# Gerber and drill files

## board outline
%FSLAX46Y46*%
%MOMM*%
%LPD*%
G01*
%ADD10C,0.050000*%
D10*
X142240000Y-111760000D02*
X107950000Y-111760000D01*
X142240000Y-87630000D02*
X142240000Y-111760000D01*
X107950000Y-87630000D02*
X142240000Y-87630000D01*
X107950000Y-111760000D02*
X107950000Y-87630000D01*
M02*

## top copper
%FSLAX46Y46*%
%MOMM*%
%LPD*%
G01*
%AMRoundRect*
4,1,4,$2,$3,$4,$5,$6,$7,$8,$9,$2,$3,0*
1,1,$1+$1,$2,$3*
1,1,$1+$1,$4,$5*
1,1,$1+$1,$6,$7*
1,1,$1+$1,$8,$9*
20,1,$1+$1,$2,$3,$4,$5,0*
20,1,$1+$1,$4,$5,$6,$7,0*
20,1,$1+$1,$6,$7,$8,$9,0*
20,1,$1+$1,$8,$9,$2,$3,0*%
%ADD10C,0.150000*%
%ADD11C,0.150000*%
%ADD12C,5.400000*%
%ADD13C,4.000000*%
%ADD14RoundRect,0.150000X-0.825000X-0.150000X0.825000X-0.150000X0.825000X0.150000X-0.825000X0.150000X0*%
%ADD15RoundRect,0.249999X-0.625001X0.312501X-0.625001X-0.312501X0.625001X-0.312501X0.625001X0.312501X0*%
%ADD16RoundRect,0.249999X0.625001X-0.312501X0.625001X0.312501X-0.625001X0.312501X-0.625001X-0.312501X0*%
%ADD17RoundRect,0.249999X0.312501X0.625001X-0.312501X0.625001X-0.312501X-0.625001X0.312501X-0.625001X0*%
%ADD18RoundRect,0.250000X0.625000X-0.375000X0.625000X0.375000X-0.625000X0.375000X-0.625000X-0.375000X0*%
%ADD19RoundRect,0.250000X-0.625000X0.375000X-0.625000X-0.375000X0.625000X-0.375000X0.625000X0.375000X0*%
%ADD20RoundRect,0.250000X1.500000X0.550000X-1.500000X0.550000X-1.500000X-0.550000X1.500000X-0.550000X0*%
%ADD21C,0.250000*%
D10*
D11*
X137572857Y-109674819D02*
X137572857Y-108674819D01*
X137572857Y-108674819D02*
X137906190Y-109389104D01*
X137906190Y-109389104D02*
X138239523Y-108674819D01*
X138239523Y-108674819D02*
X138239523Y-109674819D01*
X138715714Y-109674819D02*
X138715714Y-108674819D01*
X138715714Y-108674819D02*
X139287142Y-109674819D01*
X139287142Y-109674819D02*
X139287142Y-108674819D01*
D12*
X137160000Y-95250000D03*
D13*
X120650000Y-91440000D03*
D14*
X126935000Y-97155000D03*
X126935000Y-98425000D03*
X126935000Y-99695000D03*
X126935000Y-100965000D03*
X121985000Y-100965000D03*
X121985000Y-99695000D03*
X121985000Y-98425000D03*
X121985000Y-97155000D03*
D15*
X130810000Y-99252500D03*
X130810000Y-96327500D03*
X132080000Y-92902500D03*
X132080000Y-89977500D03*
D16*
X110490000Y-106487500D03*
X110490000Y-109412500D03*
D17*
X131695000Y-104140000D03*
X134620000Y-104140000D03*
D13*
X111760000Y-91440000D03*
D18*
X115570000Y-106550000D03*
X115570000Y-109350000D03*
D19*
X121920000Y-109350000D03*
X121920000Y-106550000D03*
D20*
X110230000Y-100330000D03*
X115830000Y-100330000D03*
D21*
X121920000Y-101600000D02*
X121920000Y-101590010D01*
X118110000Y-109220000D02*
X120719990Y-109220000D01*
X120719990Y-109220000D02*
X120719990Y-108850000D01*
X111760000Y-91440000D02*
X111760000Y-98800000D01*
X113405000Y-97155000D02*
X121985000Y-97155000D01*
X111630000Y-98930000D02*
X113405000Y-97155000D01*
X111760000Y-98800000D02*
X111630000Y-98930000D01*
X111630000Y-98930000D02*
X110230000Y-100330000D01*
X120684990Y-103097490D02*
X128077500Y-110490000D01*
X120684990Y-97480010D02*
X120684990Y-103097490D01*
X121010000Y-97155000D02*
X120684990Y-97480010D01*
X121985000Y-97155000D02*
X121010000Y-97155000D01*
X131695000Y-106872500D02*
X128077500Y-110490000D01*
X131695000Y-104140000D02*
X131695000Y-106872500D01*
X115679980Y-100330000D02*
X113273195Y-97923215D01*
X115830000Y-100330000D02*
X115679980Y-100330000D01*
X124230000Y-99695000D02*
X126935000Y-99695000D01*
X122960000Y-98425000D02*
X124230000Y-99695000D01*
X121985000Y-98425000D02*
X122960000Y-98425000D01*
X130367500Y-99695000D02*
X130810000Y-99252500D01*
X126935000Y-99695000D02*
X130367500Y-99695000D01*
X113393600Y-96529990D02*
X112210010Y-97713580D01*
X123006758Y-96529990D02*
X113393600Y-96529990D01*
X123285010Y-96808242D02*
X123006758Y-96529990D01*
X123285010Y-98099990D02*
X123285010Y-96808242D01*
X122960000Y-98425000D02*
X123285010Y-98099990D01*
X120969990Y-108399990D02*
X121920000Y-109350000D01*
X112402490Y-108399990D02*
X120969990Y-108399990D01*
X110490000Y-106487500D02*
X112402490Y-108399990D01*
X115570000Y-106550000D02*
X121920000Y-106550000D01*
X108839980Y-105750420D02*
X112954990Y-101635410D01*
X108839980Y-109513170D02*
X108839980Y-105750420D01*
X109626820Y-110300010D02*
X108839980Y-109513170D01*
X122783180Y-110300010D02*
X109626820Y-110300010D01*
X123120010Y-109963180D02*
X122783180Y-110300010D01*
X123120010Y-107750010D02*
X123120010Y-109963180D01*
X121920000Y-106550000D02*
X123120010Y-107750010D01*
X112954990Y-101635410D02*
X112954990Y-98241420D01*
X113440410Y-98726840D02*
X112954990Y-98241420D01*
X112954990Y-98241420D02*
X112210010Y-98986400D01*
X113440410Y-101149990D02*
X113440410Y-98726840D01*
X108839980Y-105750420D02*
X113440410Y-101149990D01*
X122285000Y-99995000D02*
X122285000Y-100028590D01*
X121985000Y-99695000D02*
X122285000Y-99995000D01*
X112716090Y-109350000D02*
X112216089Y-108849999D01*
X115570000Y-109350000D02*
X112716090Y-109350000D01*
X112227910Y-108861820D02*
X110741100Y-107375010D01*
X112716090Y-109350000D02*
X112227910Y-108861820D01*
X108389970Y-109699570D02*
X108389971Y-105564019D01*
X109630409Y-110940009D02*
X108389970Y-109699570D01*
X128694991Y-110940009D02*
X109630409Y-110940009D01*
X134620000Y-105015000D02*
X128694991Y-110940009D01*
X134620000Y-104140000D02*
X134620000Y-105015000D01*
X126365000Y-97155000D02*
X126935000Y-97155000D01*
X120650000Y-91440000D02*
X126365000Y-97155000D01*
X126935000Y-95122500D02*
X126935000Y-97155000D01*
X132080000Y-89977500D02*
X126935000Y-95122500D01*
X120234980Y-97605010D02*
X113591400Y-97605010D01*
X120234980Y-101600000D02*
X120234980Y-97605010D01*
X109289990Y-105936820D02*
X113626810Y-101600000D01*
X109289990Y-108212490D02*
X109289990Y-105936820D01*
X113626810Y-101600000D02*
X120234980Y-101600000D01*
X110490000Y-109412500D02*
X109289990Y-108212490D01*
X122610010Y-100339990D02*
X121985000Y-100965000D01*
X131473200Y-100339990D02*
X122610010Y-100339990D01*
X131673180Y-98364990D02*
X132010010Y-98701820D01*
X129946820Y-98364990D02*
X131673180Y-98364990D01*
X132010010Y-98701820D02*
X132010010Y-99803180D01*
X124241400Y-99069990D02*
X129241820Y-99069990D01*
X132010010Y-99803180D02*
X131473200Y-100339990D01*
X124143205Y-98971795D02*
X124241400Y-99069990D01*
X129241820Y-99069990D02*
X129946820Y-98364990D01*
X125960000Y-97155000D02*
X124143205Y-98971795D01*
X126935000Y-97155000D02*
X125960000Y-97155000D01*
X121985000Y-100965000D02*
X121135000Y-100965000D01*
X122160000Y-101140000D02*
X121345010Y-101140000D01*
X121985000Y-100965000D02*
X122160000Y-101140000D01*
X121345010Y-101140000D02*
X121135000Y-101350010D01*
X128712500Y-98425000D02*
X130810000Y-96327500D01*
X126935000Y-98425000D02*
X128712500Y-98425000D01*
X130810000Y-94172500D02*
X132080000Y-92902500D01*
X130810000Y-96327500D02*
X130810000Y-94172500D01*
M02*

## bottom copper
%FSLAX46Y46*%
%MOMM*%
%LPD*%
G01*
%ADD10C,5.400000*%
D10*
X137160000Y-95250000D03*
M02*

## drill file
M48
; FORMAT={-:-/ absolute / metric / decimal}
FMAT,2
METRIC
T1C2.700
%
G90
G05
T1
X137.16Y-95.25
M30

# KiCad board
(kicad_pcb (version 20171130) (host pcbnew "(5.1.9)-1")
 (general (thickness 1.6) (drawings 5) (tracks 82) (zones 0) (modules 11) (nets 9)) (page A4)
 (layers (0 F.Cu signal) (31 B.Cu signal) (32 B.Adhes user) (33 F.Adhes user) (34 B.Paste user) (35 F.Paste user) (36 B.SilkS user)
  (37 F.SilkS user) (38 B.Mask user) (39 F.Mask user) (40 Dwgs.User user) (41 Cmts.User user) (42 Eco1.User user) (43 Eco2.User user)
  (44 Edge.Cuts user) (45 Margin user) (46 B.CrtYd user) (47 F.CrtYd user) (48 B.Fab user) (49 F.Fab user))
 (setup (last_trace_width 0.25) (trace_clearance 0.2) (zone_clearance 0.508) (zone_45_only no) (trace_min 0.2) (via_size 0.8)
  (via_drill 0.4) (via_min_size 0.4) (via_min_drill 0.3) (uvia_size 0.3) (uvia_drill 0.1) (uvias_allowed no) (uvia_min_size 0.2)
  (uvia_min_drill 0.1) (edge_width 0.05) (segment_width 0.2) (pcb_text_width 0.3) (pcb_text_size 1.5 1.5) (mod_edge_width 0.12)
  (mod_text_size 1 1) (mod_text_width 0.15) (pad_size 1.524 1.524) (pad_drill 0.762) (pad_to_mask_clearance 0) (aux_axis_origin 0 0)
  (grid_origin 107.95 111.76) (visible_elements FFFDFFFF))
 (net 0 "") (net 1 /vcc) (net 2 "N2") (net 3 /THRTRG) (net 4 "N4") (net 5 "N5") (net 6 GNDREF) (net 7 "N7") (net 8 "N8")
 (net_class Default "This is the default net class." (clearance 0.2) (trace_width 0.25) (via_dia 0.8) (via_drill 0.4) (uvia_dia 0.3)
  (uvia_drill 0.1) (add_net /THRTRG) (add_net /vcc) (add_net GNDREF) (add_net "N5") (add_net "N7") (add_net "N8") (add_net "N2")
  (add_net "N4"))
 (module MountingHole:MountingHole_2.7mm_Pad (layer F.Cu) (at 137.16 95.25)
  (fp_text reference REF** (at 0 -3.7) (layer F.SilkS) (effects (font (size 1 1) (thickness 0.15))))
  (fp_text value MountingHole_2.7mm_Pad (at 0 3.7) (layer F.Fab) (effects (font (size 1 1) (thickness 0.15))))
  (pad 1 thru_hole circle (at 0 0) (size 5.4 5.4) (drill 2.7) (layers *.Cu *.Mask)))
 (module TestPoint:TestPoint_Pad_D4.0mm (layer F.Cu) (at 120.65 91.44)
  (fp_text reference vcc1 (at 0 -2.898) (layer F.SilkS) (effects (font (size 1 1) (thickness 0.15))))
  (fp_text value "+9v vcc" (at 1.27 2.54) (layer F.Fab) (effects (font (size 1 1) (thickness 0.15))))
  (pad 1 smd circle (at 0 0) (size 4 4) (layers F.Cu F.Mask) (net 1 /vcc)))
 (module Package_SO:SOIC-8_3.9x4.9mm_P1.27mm (layer F.Cu) (at 124.46 99.06)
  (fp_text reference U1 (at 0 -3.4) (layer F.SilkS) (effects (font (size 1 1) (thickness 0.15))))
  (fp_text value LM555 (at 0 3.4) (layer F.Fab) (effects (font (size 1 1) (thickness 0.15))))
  (pad 8 smd roundrect (at 2.475 -1.905) (size 1.95 0.6) (layers F.Cu F.Paste F.Mask) (roundrect_rratio 0.25) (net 1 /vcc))
  (pad 7 smd roundrect (at 2.475 -0.635) (size 1.95 0.6) (layers F.Cu F.Paste F.Mask) (roundrect_rratio 0.25) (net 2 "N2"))
  (pad 6 smd roundrect (at 2.475 0.635) (size 1.95 0.6) (layers F.Cu F.Paste F.Mask) (roundrect_rratio 0.25) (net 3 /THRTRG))
  (pad 5 smd roundrect (at 2.475 1.905) (size 1.95 0.6) (layers F.Cu F.Paste F.Mask) (roundrect_rratio 0.25) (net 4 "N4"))
  (pad 4 smd roundrect (at -2.475 1.905) (size 1.95 0.6) (layers F.Cu F.Paste F.Mask) (roundrect_rratio 0.25) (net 1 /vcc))
  (pad 3 smd roundrect (at -2.475 0.635) (size 1.95 0.6) (layers F.Cu F.Paste F.Mask) (roundrect_rratio 0.25) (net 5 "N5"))
  (pad 2 smd roundrect (at -2.475 -0.635) (size 1.95 0.6) (layers F.Cu F.Paste F.Mask) (roundrect_rratio 0.25) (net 3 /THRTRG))
  (pad 1 smd roundrect (at -2.475 -1.905) (size 1.95 0.6) (layers F.Cu F.Paste F.Mask) (roundrect_rratio 0.25) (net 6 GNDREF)))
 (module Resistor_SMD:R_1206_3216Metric (layer F.Cu) (at 130.81 97.79 270)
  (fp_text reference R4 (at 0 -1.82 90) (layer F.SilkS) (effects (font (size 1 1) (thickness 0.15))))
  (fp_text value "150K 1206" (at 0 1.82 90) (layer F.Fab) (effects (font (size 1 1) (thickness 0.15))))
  (pad 2 smd roundrect (at 1.4625 0 270) (size 1.125 1.75) (layers F.Cu F.Paste F.Mask) (roundrect_rratio 0.2222213333333333)
   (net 3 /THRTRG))
  (pad 1 smd roundrect (at -1.4625 0 270) (size 1.125 1.75) (layers F.Cu F.Paste F.Mask) (roundrect_rratio 0.2222213333333333) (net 2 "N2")))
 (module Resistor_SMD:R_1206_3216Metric (layer F.Cu) (at 132.08 91.44 270)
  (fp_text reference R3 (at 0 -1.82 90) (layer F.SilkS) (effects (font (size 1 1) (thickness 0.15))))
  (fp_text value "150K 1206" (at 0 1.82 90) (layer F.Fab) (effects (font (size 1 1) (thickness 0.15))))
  (pad 2 smd roundrect (at 1.4625 0 270) (size 1.125 1.75) (layers F.Cu F.Paste F.Mask) (roundrect_rratio 0.2222213333333333) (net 2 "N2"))
  (pad 1 smd roundrect (at -1.4625 0 270) (size 1.125 1.75) (layers F.Cu F.Paste F.Mask) (roundrect_rratio 0.2222213333333333) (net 1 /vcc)))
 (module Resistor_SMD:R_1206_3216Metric (layer F.Cu) (at 110.49 107.95 90)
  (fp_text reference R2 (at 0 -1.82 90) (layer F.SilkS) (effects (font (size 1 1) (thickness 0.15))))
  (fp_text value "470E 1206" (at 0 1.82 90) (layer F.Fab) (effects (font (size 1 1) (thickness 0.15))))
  (pad 2 smd roundrect (at 1.4625 0 90) (size 1.125 1.75) (layers F.Cu F.Paste F.Mask) (roundrect_rratio 0.2222213333333333) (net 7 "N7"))
  (pad 1 smd roundrect (at -1.4625 0 90) (size 1.125 1.75) (layers F.Cu F.Paste F.Mask) (roundrect_rratio 0.2222213333333333) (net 1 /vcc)))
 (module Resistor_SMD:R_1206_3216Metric (layer F.Cu) (at 133.1575 104.14 180)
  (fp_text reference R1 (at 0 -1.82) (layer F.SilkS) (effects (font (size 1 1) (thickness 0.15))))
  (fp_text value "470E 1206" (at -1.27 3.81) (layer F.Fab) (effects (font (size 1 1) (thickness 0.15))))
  (pad 2 smd roundrect (at 1.4625 0 180) (size 1.125 1.75) (layers F.Cu F.Paste F.Mask) (roundrect_rratio 0.2222213333333333) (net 6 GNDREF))
  (pad 1 smd roundrect (at -1.4625 0 180) (size 1.125 1.75) (layers F.Cu F.Paste F.Mask) (roundrect_rratio 0.2222213333333333) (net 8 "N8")))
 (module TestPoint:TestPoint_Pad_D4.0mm (layer F.Cu) (at 111.76 91.44)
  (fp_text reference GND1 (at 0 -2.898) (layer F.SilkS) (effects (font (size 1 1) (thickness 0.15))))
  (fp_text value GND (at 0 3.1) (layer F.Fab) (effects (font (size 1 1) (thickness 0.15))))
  (pad 1 smd circle (at 0 0) (size 4 4) (layers F.Cu F.Mask) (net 6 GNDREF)))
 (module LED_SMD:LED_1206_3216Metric (layer F.Cu) (at 115.57 107.95 90)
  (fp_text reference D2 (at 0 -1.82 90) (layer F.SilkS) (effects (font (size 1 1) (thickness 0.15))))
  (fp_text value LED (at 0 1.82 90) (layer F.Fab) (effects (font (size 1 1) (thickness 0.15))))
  (pad 2 smd roundrect (at 1.4 0 90) (size 1.25 1.75) (layers F.Cu F.Paste F.Mask) (roundrect_rratio 0.2) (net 5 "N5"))
  (pad 1 smd roundrect (at -1.4 0 90) (size 1.25 1.75) (layers F.Cu F.Paste F.Mask) (roundrect_rratio 0.2) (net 8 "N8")))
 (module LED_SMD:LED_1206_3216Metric (layer F.Cu) (at 121.92 107.95 270)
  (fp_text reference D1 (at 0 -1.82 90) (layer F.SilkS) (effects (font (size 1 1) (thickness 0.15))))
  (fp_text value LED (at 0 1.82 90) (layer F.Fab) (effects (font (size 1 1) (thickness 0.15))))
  (pad 2 smd roundrect (at 1.4 0 270) (size 1.25 1.75) (layers F.Cu F.Paste F.Mask) (roundrect_rratio 0.2) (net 7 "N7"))
  (pad 1 smd roundrect (at -1.4 0 270) (size 1.25 1.75) (layers F.Cu F.Paste F.Mask) (roundrect_rratio 0.2) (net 5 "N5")))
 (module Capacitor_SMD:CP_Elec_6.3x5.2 (layer F.Cu) (at 113.03 100.33 180)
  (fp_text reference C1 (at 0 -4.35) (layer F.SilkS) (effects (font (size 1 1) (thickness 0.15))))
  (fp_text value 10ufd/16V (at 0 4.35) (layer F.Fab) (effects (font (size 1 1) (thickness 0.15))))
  (pad 2 smd roundrect (at 2.8 0 180) (size 3.5 1.6) (layers F.Cu F.Paste F.Mask) (roundrect_rratio 0.15625) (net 6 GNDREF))
  (pad 1 smd roundrect (at -2.8 0 180) (size 3.5 1.6) (layers F.Cu F.Paste F.Mask) (roundrect_rratio 0.15625) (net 3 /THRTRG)))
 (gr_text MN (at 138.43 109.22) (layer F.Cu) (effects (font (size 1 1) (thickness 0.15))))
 (gr_line (start 142.24 111.76) (end 107.95 111.76) (layer Edge.Cuts) (width 0.05))
 (gr_line (start 142.24 87.63) (end 142.24 111.76) (layer Edge.Cuts) (width 0.05))
 (gr_line (start 107.95 87.63) (end 142.24 87.63) (layer Edge.Cuts) (width 0.05))
 (gr_line (start 107.95 111.76) (end 107.95 87.63) (layer Edge.Cuts) (width 0.05))
 (segment (start 121.92 101.6) (end 121.92 101.59001) (width 0.25) (layer F.Cu) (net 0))
 (segment (start 118.11 109.22) (end 120.71999 109.22) (width 0.25) (layer F.Cu) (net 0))
 (segment (start 120.71999 109.22) (end 120.71999 108.85) (width 0.25) (layer F.Cu) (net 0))
 (segment (start 111.76 91.44) (end 111.76 98.8) (width 0.25) (layer F.Cu) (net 6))
 (segment (start 113.405 97.155) (end 121.985 97.155) (width 0.25) (layer F.Cu) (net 6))
 (segment (start 111.63 98.93) (end 113.405 97.155) (width 0.25) (layer F.Cu) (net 6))
 (segment (start 111.76 98.8) (end 111.63 98.93) (width 0.25) (layer F.Cu) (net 6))
 (segment (start 111.63 98.93) (end 110.23 100.33) (width 0.25) (layer F.Cu) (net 6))
 (segment (start 120.68499 103.09749) (end 128.0775 110.49) (width 0.25) (layer F.Cu) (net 6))
 (segment (start 120.68499 97.48001) (end 120.68499 103.09749) (width 0.25) (layer F.Cu) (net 6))
 (segment (start 121.01 97.155) (end 120.68499 97.48001) (width 0.25) (layer F.Cu) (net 6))
 (segment (start 121.985 97.155) (end 121.01 97.155) (width 0.25) (layer F.Cu) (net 6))
 (segment (start 131.695 106.8725) (end 128.0775 110.49) (width 0.25) (layer F.Cu) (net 6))
 (segment (start 131.695 104.14) (end 131.695 106.8725) (width 0.25) (layer F.Cu) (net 6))
 (segment (start 115.67998 100.33) (end 113.273195 97.923215) (width 0.25) (layer F.Cu) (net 3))
 (segment (start 115.83 100.33) (end 115.67998 100.33) (width 0.25) (layer F.Cu) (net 3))
 (segment (start 124.23 99.695) (end 126.935 99.695) (width 0.25) (layer F.Cu) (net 3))
 (segment (start 122.96 98.425) (end 124.23 99.695) (width 0.25) (layer F.Cu) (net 3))
 (segment (start 121.985 98.425) (end 122.96 98.425) (width 0.25) (layer F.Cu) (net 3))
 (segment (start 130.3675 99.695) (end 130.81 99.2525) (width 0.25) (layer F.Cu) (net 3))
 (segment (start 126.935 99.695) (end 130.3675 99.695) (width 0.25) (layer F.Cu) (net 3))
 (segment (start 113.3936 96.52999) (end 112.21001 97.71358) (width 0.25) (layer F.Cu) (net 3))
 (segment (start 123.006758 96.52999) (end 113.3936 96.52999) (width 0.25) (layer F.Cu) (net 3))
 (segment (start 123.28501 96.808242) (end 123.006758 96.52999) (width 0.25) (layer F.Cu) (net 3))
 (segment (start 123.28501 98.09999) (end 123.28501 96.808242) (width 0.25) (layer F.Cu) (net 3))
 (segment (start 122.96 98.425) (end 123.28501 98.09999) (width 0.25) (layer F.Cu) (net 3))
 (segment (start 120.96999 108.39999) (end 121.92 109.35) (width 0.25) (layer F.Cu) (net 7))
 (segment (start 112.40249 108.39999) (end 120.96999 108.39999) (width 0.25) (layer F.Cu) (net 7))
 (segment (start 110.49 106.4875) (end 112.40249 108.39999) (width 0.25) (layer F.Cu) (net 7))
 (segment (start 115.57 106.55) (end 121.92 106.55) (width 0.25) (layer F.Cu) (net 5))
 (segment (start 108.83998 105.75042) (end 112.95499 101.63541) (width 0.25) (layer F.Cu) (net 5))
 (segment (start 108.83998 109.51317) (end 108.83998 105.75042) (width 0.25) (layer F.Cu) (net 5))
 (segment (start 109.62682 110.30001) (end 108.83998 109.51317) (width 0.25) (layer F.Cu) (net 5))
 (segment (start 122.78318 110.30001) (end 109.62682 110.30001) (width 0.25) (layer F.Cu) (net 5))
 (segment (start 123.12001 109.96318) (end 122.78318 110.30001) (width 0.25) (layer F.Cu) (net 5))
 (segment (start 123.12001 107.75001) (end 123.12001 109.96318) (width 0.25) (layer F.Cu) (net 5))
 (segment (start 121.92 106.55) (end 123.12001 107.75001) (width 0.25) (layer F.Cu) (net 5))
 (segment (start 112.95499 101.63541) (end 112.95499 98.24142) (width 0.25) (layer F.Cu) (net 5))
 (segment (start 113.44041 98.72684) (end 112.95499 98.24142) (width 0.25) (layer F.Cu) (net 5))
 (segment (start 112.95499 98.24142) (end 112.21001 98.9864) (width 0.25) (layer F.Cu) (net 5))
 (segment (start 113.44041 101.14999) (end 113.44041 98.72684) (width 0.25) (layer F.Cu) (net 5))
 (segment (start 108.83998 105.75042) (end 113.44041 101.14999) (width 0.25) (layer F.Cu) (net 5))
 (segment (start 122.285 99.995) (end 122.285 100.02859) (width 0.25) (layer F.Cu) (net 5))
 (segment (start 121.985 99.695) (end 122.285 99.995) (width 0.25) (layer F.Cu) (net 5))
 (segment (start 112.71609 109.35) (end 112.216089 108.849999) (width 0.25) (layer F.Cu) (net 8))
 (segment (start 115.57 109.35) (end 112.71609 109.35) (width 0.25) (layer F.Cu) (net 8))
 (segment (start 112.22791 108.86182) (end 110.7411 107.37501) (width 0.25) (layer F.Cu) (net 8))
 (segment (start 112.71609 109.35) (end 112.22791 108.86182) (width 0.25) (layer F.Cu) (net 8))
 (segment (start 108.38997 109.69957) (end 108.389971 105.564019) (width 0.25) (layer F.Cu) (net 8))
 (segment (start 109.630409 110.940009) (end 108.38997 109.69957) (width 0.25) (layer F.Cu) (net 8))
 (segment (start 128.694991 110.940009) (end 109.630409 110.940009) (width 0.25) (layer F.Cu) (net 8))
 (segment (start 134.62 105.015) (end 128.694991 110.940009) (width 0.25) (layer F.Cu) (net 8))
 (segment (start 134.62 104.14) (end 134.62 105.015) (width 0.25) (layer F.Cu) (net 8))
 (segment (start 126.365 97.155) (end 126.935 97.155) (width 0.25) (layer F.Cu) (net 1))
 (segment (start 120.65 91.44) (end 126.365 97.155) (width 0.25) (layer F.Cu) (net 1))
 (segment (start 126.935 95.1225) (end 126.935 97.155) (width 0.25) (layer F.Cu) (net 1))
 (segment (start 132.08 89.9775) (end 126.935 95.1225) (width 0.25) (layer F.Cu) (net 1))
 (segment (start 120.23498 97.60501) (end 113.5914 97.60501) (width 0.25) (layer F.Cu) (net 1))
 (segment (start 120.23498 101.6) (end 120.23498 97.60501) (width 0.25) (layer F.Cu) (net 1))
 (segment (start 109.28999 105.93682) (end 113.62681 101.6) (width 0.25) (layer F.Cu) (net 1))
 (segment (start 109.28999 108.21249) (end 109.28999 105.93682) (width 0.25) (layer F.Cu) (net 1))
 (segment (start 113.62681 101.6) (end 120.23498 101.6) (width 0.25) (layer F.Cu) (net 1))
 (segment (start 110.49 109.4125) (end 109.28999 108.21249) (width 0.25) (layer F.Cu) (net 1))
 (segment (start 122.61001 100.33999) (end 121.985 100.965) (width 0.25) (layer F.Cu) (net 1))
 (segment (start 131.4732 100.33999) (end 122.61001 100.33999) (width 0.25) (layer F.Cu) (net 1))
 (segment (start 131.67318 98.36499) (end 132.01001 98.70182) (width 0.25) (layer F.Cu) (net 1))
 (segment (start 129.94682 98.36499) (end 131.67318 98.36499) (width 0.25) (layer F.Cu) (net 1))
 (segment (start 132.01001 98.70182) (end 132.01001 99.80318) (width 0.25) (layer F.Cu) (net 1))
 (segment (start 124.2414 99.06999) (end 129.24182 99.06999) (width 0.25) (layer F.Cu) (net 1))
 (segment (start 132.01001 99.80318) (end 131.4732 100.33999) (width 0.25) (layer F.Cu) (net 1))
 (segment (start 124.143205 98.971795) (end 124.2414 99.06999) (width 0.25) (layer F.Cu) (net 1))
 (segment (start 129.24182 99.06999) (end 129.94682 98.36499) (width 0.25) (layer F.Cu) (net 1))
 (segment (start 125.96 97.155) (end 124.143205 98.971795) (width 0.25) (layer F.Cu) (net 1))
 (segment (start 126.935 97.155) (end 125.96 97.155) (width 0.25) (layer F.Cu) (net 1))
 (segment (start 121.985 100.965) (end 121.135 100.965) (width 0.25) (layer F.Cu) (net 1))
 (segment (start 122.16 101.14) (end 121.34501 101.14) (width 0.25) (layer F.Cu) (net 1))
 (segment (start 121.985 100.965) (end 122.16 101.14) (width 0.25) (layer F.Cu) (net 1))
 (segment (start 121.34501 101.14) (end 121.135 101.35001) (width 0.25) (layer F.Cu) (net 1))
 (segment (start 128.7125 98.425) (end 130.81 96.3275) (width 0.25) (layer F.Cu) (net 2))
 (segment (start 126.935 98.425) (end 128.7125 98.425) (width 0.25) (layer F.Cu) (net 2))
 (segment (start 130.81 94.1725) (end 132.08 92.9025) (width 0.25) (layer F.Cu) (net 2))
 (segment (start 130.81 96.3275) (end 130.81 94.1725) (width 0.25) (layer F.Cu) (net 2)))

